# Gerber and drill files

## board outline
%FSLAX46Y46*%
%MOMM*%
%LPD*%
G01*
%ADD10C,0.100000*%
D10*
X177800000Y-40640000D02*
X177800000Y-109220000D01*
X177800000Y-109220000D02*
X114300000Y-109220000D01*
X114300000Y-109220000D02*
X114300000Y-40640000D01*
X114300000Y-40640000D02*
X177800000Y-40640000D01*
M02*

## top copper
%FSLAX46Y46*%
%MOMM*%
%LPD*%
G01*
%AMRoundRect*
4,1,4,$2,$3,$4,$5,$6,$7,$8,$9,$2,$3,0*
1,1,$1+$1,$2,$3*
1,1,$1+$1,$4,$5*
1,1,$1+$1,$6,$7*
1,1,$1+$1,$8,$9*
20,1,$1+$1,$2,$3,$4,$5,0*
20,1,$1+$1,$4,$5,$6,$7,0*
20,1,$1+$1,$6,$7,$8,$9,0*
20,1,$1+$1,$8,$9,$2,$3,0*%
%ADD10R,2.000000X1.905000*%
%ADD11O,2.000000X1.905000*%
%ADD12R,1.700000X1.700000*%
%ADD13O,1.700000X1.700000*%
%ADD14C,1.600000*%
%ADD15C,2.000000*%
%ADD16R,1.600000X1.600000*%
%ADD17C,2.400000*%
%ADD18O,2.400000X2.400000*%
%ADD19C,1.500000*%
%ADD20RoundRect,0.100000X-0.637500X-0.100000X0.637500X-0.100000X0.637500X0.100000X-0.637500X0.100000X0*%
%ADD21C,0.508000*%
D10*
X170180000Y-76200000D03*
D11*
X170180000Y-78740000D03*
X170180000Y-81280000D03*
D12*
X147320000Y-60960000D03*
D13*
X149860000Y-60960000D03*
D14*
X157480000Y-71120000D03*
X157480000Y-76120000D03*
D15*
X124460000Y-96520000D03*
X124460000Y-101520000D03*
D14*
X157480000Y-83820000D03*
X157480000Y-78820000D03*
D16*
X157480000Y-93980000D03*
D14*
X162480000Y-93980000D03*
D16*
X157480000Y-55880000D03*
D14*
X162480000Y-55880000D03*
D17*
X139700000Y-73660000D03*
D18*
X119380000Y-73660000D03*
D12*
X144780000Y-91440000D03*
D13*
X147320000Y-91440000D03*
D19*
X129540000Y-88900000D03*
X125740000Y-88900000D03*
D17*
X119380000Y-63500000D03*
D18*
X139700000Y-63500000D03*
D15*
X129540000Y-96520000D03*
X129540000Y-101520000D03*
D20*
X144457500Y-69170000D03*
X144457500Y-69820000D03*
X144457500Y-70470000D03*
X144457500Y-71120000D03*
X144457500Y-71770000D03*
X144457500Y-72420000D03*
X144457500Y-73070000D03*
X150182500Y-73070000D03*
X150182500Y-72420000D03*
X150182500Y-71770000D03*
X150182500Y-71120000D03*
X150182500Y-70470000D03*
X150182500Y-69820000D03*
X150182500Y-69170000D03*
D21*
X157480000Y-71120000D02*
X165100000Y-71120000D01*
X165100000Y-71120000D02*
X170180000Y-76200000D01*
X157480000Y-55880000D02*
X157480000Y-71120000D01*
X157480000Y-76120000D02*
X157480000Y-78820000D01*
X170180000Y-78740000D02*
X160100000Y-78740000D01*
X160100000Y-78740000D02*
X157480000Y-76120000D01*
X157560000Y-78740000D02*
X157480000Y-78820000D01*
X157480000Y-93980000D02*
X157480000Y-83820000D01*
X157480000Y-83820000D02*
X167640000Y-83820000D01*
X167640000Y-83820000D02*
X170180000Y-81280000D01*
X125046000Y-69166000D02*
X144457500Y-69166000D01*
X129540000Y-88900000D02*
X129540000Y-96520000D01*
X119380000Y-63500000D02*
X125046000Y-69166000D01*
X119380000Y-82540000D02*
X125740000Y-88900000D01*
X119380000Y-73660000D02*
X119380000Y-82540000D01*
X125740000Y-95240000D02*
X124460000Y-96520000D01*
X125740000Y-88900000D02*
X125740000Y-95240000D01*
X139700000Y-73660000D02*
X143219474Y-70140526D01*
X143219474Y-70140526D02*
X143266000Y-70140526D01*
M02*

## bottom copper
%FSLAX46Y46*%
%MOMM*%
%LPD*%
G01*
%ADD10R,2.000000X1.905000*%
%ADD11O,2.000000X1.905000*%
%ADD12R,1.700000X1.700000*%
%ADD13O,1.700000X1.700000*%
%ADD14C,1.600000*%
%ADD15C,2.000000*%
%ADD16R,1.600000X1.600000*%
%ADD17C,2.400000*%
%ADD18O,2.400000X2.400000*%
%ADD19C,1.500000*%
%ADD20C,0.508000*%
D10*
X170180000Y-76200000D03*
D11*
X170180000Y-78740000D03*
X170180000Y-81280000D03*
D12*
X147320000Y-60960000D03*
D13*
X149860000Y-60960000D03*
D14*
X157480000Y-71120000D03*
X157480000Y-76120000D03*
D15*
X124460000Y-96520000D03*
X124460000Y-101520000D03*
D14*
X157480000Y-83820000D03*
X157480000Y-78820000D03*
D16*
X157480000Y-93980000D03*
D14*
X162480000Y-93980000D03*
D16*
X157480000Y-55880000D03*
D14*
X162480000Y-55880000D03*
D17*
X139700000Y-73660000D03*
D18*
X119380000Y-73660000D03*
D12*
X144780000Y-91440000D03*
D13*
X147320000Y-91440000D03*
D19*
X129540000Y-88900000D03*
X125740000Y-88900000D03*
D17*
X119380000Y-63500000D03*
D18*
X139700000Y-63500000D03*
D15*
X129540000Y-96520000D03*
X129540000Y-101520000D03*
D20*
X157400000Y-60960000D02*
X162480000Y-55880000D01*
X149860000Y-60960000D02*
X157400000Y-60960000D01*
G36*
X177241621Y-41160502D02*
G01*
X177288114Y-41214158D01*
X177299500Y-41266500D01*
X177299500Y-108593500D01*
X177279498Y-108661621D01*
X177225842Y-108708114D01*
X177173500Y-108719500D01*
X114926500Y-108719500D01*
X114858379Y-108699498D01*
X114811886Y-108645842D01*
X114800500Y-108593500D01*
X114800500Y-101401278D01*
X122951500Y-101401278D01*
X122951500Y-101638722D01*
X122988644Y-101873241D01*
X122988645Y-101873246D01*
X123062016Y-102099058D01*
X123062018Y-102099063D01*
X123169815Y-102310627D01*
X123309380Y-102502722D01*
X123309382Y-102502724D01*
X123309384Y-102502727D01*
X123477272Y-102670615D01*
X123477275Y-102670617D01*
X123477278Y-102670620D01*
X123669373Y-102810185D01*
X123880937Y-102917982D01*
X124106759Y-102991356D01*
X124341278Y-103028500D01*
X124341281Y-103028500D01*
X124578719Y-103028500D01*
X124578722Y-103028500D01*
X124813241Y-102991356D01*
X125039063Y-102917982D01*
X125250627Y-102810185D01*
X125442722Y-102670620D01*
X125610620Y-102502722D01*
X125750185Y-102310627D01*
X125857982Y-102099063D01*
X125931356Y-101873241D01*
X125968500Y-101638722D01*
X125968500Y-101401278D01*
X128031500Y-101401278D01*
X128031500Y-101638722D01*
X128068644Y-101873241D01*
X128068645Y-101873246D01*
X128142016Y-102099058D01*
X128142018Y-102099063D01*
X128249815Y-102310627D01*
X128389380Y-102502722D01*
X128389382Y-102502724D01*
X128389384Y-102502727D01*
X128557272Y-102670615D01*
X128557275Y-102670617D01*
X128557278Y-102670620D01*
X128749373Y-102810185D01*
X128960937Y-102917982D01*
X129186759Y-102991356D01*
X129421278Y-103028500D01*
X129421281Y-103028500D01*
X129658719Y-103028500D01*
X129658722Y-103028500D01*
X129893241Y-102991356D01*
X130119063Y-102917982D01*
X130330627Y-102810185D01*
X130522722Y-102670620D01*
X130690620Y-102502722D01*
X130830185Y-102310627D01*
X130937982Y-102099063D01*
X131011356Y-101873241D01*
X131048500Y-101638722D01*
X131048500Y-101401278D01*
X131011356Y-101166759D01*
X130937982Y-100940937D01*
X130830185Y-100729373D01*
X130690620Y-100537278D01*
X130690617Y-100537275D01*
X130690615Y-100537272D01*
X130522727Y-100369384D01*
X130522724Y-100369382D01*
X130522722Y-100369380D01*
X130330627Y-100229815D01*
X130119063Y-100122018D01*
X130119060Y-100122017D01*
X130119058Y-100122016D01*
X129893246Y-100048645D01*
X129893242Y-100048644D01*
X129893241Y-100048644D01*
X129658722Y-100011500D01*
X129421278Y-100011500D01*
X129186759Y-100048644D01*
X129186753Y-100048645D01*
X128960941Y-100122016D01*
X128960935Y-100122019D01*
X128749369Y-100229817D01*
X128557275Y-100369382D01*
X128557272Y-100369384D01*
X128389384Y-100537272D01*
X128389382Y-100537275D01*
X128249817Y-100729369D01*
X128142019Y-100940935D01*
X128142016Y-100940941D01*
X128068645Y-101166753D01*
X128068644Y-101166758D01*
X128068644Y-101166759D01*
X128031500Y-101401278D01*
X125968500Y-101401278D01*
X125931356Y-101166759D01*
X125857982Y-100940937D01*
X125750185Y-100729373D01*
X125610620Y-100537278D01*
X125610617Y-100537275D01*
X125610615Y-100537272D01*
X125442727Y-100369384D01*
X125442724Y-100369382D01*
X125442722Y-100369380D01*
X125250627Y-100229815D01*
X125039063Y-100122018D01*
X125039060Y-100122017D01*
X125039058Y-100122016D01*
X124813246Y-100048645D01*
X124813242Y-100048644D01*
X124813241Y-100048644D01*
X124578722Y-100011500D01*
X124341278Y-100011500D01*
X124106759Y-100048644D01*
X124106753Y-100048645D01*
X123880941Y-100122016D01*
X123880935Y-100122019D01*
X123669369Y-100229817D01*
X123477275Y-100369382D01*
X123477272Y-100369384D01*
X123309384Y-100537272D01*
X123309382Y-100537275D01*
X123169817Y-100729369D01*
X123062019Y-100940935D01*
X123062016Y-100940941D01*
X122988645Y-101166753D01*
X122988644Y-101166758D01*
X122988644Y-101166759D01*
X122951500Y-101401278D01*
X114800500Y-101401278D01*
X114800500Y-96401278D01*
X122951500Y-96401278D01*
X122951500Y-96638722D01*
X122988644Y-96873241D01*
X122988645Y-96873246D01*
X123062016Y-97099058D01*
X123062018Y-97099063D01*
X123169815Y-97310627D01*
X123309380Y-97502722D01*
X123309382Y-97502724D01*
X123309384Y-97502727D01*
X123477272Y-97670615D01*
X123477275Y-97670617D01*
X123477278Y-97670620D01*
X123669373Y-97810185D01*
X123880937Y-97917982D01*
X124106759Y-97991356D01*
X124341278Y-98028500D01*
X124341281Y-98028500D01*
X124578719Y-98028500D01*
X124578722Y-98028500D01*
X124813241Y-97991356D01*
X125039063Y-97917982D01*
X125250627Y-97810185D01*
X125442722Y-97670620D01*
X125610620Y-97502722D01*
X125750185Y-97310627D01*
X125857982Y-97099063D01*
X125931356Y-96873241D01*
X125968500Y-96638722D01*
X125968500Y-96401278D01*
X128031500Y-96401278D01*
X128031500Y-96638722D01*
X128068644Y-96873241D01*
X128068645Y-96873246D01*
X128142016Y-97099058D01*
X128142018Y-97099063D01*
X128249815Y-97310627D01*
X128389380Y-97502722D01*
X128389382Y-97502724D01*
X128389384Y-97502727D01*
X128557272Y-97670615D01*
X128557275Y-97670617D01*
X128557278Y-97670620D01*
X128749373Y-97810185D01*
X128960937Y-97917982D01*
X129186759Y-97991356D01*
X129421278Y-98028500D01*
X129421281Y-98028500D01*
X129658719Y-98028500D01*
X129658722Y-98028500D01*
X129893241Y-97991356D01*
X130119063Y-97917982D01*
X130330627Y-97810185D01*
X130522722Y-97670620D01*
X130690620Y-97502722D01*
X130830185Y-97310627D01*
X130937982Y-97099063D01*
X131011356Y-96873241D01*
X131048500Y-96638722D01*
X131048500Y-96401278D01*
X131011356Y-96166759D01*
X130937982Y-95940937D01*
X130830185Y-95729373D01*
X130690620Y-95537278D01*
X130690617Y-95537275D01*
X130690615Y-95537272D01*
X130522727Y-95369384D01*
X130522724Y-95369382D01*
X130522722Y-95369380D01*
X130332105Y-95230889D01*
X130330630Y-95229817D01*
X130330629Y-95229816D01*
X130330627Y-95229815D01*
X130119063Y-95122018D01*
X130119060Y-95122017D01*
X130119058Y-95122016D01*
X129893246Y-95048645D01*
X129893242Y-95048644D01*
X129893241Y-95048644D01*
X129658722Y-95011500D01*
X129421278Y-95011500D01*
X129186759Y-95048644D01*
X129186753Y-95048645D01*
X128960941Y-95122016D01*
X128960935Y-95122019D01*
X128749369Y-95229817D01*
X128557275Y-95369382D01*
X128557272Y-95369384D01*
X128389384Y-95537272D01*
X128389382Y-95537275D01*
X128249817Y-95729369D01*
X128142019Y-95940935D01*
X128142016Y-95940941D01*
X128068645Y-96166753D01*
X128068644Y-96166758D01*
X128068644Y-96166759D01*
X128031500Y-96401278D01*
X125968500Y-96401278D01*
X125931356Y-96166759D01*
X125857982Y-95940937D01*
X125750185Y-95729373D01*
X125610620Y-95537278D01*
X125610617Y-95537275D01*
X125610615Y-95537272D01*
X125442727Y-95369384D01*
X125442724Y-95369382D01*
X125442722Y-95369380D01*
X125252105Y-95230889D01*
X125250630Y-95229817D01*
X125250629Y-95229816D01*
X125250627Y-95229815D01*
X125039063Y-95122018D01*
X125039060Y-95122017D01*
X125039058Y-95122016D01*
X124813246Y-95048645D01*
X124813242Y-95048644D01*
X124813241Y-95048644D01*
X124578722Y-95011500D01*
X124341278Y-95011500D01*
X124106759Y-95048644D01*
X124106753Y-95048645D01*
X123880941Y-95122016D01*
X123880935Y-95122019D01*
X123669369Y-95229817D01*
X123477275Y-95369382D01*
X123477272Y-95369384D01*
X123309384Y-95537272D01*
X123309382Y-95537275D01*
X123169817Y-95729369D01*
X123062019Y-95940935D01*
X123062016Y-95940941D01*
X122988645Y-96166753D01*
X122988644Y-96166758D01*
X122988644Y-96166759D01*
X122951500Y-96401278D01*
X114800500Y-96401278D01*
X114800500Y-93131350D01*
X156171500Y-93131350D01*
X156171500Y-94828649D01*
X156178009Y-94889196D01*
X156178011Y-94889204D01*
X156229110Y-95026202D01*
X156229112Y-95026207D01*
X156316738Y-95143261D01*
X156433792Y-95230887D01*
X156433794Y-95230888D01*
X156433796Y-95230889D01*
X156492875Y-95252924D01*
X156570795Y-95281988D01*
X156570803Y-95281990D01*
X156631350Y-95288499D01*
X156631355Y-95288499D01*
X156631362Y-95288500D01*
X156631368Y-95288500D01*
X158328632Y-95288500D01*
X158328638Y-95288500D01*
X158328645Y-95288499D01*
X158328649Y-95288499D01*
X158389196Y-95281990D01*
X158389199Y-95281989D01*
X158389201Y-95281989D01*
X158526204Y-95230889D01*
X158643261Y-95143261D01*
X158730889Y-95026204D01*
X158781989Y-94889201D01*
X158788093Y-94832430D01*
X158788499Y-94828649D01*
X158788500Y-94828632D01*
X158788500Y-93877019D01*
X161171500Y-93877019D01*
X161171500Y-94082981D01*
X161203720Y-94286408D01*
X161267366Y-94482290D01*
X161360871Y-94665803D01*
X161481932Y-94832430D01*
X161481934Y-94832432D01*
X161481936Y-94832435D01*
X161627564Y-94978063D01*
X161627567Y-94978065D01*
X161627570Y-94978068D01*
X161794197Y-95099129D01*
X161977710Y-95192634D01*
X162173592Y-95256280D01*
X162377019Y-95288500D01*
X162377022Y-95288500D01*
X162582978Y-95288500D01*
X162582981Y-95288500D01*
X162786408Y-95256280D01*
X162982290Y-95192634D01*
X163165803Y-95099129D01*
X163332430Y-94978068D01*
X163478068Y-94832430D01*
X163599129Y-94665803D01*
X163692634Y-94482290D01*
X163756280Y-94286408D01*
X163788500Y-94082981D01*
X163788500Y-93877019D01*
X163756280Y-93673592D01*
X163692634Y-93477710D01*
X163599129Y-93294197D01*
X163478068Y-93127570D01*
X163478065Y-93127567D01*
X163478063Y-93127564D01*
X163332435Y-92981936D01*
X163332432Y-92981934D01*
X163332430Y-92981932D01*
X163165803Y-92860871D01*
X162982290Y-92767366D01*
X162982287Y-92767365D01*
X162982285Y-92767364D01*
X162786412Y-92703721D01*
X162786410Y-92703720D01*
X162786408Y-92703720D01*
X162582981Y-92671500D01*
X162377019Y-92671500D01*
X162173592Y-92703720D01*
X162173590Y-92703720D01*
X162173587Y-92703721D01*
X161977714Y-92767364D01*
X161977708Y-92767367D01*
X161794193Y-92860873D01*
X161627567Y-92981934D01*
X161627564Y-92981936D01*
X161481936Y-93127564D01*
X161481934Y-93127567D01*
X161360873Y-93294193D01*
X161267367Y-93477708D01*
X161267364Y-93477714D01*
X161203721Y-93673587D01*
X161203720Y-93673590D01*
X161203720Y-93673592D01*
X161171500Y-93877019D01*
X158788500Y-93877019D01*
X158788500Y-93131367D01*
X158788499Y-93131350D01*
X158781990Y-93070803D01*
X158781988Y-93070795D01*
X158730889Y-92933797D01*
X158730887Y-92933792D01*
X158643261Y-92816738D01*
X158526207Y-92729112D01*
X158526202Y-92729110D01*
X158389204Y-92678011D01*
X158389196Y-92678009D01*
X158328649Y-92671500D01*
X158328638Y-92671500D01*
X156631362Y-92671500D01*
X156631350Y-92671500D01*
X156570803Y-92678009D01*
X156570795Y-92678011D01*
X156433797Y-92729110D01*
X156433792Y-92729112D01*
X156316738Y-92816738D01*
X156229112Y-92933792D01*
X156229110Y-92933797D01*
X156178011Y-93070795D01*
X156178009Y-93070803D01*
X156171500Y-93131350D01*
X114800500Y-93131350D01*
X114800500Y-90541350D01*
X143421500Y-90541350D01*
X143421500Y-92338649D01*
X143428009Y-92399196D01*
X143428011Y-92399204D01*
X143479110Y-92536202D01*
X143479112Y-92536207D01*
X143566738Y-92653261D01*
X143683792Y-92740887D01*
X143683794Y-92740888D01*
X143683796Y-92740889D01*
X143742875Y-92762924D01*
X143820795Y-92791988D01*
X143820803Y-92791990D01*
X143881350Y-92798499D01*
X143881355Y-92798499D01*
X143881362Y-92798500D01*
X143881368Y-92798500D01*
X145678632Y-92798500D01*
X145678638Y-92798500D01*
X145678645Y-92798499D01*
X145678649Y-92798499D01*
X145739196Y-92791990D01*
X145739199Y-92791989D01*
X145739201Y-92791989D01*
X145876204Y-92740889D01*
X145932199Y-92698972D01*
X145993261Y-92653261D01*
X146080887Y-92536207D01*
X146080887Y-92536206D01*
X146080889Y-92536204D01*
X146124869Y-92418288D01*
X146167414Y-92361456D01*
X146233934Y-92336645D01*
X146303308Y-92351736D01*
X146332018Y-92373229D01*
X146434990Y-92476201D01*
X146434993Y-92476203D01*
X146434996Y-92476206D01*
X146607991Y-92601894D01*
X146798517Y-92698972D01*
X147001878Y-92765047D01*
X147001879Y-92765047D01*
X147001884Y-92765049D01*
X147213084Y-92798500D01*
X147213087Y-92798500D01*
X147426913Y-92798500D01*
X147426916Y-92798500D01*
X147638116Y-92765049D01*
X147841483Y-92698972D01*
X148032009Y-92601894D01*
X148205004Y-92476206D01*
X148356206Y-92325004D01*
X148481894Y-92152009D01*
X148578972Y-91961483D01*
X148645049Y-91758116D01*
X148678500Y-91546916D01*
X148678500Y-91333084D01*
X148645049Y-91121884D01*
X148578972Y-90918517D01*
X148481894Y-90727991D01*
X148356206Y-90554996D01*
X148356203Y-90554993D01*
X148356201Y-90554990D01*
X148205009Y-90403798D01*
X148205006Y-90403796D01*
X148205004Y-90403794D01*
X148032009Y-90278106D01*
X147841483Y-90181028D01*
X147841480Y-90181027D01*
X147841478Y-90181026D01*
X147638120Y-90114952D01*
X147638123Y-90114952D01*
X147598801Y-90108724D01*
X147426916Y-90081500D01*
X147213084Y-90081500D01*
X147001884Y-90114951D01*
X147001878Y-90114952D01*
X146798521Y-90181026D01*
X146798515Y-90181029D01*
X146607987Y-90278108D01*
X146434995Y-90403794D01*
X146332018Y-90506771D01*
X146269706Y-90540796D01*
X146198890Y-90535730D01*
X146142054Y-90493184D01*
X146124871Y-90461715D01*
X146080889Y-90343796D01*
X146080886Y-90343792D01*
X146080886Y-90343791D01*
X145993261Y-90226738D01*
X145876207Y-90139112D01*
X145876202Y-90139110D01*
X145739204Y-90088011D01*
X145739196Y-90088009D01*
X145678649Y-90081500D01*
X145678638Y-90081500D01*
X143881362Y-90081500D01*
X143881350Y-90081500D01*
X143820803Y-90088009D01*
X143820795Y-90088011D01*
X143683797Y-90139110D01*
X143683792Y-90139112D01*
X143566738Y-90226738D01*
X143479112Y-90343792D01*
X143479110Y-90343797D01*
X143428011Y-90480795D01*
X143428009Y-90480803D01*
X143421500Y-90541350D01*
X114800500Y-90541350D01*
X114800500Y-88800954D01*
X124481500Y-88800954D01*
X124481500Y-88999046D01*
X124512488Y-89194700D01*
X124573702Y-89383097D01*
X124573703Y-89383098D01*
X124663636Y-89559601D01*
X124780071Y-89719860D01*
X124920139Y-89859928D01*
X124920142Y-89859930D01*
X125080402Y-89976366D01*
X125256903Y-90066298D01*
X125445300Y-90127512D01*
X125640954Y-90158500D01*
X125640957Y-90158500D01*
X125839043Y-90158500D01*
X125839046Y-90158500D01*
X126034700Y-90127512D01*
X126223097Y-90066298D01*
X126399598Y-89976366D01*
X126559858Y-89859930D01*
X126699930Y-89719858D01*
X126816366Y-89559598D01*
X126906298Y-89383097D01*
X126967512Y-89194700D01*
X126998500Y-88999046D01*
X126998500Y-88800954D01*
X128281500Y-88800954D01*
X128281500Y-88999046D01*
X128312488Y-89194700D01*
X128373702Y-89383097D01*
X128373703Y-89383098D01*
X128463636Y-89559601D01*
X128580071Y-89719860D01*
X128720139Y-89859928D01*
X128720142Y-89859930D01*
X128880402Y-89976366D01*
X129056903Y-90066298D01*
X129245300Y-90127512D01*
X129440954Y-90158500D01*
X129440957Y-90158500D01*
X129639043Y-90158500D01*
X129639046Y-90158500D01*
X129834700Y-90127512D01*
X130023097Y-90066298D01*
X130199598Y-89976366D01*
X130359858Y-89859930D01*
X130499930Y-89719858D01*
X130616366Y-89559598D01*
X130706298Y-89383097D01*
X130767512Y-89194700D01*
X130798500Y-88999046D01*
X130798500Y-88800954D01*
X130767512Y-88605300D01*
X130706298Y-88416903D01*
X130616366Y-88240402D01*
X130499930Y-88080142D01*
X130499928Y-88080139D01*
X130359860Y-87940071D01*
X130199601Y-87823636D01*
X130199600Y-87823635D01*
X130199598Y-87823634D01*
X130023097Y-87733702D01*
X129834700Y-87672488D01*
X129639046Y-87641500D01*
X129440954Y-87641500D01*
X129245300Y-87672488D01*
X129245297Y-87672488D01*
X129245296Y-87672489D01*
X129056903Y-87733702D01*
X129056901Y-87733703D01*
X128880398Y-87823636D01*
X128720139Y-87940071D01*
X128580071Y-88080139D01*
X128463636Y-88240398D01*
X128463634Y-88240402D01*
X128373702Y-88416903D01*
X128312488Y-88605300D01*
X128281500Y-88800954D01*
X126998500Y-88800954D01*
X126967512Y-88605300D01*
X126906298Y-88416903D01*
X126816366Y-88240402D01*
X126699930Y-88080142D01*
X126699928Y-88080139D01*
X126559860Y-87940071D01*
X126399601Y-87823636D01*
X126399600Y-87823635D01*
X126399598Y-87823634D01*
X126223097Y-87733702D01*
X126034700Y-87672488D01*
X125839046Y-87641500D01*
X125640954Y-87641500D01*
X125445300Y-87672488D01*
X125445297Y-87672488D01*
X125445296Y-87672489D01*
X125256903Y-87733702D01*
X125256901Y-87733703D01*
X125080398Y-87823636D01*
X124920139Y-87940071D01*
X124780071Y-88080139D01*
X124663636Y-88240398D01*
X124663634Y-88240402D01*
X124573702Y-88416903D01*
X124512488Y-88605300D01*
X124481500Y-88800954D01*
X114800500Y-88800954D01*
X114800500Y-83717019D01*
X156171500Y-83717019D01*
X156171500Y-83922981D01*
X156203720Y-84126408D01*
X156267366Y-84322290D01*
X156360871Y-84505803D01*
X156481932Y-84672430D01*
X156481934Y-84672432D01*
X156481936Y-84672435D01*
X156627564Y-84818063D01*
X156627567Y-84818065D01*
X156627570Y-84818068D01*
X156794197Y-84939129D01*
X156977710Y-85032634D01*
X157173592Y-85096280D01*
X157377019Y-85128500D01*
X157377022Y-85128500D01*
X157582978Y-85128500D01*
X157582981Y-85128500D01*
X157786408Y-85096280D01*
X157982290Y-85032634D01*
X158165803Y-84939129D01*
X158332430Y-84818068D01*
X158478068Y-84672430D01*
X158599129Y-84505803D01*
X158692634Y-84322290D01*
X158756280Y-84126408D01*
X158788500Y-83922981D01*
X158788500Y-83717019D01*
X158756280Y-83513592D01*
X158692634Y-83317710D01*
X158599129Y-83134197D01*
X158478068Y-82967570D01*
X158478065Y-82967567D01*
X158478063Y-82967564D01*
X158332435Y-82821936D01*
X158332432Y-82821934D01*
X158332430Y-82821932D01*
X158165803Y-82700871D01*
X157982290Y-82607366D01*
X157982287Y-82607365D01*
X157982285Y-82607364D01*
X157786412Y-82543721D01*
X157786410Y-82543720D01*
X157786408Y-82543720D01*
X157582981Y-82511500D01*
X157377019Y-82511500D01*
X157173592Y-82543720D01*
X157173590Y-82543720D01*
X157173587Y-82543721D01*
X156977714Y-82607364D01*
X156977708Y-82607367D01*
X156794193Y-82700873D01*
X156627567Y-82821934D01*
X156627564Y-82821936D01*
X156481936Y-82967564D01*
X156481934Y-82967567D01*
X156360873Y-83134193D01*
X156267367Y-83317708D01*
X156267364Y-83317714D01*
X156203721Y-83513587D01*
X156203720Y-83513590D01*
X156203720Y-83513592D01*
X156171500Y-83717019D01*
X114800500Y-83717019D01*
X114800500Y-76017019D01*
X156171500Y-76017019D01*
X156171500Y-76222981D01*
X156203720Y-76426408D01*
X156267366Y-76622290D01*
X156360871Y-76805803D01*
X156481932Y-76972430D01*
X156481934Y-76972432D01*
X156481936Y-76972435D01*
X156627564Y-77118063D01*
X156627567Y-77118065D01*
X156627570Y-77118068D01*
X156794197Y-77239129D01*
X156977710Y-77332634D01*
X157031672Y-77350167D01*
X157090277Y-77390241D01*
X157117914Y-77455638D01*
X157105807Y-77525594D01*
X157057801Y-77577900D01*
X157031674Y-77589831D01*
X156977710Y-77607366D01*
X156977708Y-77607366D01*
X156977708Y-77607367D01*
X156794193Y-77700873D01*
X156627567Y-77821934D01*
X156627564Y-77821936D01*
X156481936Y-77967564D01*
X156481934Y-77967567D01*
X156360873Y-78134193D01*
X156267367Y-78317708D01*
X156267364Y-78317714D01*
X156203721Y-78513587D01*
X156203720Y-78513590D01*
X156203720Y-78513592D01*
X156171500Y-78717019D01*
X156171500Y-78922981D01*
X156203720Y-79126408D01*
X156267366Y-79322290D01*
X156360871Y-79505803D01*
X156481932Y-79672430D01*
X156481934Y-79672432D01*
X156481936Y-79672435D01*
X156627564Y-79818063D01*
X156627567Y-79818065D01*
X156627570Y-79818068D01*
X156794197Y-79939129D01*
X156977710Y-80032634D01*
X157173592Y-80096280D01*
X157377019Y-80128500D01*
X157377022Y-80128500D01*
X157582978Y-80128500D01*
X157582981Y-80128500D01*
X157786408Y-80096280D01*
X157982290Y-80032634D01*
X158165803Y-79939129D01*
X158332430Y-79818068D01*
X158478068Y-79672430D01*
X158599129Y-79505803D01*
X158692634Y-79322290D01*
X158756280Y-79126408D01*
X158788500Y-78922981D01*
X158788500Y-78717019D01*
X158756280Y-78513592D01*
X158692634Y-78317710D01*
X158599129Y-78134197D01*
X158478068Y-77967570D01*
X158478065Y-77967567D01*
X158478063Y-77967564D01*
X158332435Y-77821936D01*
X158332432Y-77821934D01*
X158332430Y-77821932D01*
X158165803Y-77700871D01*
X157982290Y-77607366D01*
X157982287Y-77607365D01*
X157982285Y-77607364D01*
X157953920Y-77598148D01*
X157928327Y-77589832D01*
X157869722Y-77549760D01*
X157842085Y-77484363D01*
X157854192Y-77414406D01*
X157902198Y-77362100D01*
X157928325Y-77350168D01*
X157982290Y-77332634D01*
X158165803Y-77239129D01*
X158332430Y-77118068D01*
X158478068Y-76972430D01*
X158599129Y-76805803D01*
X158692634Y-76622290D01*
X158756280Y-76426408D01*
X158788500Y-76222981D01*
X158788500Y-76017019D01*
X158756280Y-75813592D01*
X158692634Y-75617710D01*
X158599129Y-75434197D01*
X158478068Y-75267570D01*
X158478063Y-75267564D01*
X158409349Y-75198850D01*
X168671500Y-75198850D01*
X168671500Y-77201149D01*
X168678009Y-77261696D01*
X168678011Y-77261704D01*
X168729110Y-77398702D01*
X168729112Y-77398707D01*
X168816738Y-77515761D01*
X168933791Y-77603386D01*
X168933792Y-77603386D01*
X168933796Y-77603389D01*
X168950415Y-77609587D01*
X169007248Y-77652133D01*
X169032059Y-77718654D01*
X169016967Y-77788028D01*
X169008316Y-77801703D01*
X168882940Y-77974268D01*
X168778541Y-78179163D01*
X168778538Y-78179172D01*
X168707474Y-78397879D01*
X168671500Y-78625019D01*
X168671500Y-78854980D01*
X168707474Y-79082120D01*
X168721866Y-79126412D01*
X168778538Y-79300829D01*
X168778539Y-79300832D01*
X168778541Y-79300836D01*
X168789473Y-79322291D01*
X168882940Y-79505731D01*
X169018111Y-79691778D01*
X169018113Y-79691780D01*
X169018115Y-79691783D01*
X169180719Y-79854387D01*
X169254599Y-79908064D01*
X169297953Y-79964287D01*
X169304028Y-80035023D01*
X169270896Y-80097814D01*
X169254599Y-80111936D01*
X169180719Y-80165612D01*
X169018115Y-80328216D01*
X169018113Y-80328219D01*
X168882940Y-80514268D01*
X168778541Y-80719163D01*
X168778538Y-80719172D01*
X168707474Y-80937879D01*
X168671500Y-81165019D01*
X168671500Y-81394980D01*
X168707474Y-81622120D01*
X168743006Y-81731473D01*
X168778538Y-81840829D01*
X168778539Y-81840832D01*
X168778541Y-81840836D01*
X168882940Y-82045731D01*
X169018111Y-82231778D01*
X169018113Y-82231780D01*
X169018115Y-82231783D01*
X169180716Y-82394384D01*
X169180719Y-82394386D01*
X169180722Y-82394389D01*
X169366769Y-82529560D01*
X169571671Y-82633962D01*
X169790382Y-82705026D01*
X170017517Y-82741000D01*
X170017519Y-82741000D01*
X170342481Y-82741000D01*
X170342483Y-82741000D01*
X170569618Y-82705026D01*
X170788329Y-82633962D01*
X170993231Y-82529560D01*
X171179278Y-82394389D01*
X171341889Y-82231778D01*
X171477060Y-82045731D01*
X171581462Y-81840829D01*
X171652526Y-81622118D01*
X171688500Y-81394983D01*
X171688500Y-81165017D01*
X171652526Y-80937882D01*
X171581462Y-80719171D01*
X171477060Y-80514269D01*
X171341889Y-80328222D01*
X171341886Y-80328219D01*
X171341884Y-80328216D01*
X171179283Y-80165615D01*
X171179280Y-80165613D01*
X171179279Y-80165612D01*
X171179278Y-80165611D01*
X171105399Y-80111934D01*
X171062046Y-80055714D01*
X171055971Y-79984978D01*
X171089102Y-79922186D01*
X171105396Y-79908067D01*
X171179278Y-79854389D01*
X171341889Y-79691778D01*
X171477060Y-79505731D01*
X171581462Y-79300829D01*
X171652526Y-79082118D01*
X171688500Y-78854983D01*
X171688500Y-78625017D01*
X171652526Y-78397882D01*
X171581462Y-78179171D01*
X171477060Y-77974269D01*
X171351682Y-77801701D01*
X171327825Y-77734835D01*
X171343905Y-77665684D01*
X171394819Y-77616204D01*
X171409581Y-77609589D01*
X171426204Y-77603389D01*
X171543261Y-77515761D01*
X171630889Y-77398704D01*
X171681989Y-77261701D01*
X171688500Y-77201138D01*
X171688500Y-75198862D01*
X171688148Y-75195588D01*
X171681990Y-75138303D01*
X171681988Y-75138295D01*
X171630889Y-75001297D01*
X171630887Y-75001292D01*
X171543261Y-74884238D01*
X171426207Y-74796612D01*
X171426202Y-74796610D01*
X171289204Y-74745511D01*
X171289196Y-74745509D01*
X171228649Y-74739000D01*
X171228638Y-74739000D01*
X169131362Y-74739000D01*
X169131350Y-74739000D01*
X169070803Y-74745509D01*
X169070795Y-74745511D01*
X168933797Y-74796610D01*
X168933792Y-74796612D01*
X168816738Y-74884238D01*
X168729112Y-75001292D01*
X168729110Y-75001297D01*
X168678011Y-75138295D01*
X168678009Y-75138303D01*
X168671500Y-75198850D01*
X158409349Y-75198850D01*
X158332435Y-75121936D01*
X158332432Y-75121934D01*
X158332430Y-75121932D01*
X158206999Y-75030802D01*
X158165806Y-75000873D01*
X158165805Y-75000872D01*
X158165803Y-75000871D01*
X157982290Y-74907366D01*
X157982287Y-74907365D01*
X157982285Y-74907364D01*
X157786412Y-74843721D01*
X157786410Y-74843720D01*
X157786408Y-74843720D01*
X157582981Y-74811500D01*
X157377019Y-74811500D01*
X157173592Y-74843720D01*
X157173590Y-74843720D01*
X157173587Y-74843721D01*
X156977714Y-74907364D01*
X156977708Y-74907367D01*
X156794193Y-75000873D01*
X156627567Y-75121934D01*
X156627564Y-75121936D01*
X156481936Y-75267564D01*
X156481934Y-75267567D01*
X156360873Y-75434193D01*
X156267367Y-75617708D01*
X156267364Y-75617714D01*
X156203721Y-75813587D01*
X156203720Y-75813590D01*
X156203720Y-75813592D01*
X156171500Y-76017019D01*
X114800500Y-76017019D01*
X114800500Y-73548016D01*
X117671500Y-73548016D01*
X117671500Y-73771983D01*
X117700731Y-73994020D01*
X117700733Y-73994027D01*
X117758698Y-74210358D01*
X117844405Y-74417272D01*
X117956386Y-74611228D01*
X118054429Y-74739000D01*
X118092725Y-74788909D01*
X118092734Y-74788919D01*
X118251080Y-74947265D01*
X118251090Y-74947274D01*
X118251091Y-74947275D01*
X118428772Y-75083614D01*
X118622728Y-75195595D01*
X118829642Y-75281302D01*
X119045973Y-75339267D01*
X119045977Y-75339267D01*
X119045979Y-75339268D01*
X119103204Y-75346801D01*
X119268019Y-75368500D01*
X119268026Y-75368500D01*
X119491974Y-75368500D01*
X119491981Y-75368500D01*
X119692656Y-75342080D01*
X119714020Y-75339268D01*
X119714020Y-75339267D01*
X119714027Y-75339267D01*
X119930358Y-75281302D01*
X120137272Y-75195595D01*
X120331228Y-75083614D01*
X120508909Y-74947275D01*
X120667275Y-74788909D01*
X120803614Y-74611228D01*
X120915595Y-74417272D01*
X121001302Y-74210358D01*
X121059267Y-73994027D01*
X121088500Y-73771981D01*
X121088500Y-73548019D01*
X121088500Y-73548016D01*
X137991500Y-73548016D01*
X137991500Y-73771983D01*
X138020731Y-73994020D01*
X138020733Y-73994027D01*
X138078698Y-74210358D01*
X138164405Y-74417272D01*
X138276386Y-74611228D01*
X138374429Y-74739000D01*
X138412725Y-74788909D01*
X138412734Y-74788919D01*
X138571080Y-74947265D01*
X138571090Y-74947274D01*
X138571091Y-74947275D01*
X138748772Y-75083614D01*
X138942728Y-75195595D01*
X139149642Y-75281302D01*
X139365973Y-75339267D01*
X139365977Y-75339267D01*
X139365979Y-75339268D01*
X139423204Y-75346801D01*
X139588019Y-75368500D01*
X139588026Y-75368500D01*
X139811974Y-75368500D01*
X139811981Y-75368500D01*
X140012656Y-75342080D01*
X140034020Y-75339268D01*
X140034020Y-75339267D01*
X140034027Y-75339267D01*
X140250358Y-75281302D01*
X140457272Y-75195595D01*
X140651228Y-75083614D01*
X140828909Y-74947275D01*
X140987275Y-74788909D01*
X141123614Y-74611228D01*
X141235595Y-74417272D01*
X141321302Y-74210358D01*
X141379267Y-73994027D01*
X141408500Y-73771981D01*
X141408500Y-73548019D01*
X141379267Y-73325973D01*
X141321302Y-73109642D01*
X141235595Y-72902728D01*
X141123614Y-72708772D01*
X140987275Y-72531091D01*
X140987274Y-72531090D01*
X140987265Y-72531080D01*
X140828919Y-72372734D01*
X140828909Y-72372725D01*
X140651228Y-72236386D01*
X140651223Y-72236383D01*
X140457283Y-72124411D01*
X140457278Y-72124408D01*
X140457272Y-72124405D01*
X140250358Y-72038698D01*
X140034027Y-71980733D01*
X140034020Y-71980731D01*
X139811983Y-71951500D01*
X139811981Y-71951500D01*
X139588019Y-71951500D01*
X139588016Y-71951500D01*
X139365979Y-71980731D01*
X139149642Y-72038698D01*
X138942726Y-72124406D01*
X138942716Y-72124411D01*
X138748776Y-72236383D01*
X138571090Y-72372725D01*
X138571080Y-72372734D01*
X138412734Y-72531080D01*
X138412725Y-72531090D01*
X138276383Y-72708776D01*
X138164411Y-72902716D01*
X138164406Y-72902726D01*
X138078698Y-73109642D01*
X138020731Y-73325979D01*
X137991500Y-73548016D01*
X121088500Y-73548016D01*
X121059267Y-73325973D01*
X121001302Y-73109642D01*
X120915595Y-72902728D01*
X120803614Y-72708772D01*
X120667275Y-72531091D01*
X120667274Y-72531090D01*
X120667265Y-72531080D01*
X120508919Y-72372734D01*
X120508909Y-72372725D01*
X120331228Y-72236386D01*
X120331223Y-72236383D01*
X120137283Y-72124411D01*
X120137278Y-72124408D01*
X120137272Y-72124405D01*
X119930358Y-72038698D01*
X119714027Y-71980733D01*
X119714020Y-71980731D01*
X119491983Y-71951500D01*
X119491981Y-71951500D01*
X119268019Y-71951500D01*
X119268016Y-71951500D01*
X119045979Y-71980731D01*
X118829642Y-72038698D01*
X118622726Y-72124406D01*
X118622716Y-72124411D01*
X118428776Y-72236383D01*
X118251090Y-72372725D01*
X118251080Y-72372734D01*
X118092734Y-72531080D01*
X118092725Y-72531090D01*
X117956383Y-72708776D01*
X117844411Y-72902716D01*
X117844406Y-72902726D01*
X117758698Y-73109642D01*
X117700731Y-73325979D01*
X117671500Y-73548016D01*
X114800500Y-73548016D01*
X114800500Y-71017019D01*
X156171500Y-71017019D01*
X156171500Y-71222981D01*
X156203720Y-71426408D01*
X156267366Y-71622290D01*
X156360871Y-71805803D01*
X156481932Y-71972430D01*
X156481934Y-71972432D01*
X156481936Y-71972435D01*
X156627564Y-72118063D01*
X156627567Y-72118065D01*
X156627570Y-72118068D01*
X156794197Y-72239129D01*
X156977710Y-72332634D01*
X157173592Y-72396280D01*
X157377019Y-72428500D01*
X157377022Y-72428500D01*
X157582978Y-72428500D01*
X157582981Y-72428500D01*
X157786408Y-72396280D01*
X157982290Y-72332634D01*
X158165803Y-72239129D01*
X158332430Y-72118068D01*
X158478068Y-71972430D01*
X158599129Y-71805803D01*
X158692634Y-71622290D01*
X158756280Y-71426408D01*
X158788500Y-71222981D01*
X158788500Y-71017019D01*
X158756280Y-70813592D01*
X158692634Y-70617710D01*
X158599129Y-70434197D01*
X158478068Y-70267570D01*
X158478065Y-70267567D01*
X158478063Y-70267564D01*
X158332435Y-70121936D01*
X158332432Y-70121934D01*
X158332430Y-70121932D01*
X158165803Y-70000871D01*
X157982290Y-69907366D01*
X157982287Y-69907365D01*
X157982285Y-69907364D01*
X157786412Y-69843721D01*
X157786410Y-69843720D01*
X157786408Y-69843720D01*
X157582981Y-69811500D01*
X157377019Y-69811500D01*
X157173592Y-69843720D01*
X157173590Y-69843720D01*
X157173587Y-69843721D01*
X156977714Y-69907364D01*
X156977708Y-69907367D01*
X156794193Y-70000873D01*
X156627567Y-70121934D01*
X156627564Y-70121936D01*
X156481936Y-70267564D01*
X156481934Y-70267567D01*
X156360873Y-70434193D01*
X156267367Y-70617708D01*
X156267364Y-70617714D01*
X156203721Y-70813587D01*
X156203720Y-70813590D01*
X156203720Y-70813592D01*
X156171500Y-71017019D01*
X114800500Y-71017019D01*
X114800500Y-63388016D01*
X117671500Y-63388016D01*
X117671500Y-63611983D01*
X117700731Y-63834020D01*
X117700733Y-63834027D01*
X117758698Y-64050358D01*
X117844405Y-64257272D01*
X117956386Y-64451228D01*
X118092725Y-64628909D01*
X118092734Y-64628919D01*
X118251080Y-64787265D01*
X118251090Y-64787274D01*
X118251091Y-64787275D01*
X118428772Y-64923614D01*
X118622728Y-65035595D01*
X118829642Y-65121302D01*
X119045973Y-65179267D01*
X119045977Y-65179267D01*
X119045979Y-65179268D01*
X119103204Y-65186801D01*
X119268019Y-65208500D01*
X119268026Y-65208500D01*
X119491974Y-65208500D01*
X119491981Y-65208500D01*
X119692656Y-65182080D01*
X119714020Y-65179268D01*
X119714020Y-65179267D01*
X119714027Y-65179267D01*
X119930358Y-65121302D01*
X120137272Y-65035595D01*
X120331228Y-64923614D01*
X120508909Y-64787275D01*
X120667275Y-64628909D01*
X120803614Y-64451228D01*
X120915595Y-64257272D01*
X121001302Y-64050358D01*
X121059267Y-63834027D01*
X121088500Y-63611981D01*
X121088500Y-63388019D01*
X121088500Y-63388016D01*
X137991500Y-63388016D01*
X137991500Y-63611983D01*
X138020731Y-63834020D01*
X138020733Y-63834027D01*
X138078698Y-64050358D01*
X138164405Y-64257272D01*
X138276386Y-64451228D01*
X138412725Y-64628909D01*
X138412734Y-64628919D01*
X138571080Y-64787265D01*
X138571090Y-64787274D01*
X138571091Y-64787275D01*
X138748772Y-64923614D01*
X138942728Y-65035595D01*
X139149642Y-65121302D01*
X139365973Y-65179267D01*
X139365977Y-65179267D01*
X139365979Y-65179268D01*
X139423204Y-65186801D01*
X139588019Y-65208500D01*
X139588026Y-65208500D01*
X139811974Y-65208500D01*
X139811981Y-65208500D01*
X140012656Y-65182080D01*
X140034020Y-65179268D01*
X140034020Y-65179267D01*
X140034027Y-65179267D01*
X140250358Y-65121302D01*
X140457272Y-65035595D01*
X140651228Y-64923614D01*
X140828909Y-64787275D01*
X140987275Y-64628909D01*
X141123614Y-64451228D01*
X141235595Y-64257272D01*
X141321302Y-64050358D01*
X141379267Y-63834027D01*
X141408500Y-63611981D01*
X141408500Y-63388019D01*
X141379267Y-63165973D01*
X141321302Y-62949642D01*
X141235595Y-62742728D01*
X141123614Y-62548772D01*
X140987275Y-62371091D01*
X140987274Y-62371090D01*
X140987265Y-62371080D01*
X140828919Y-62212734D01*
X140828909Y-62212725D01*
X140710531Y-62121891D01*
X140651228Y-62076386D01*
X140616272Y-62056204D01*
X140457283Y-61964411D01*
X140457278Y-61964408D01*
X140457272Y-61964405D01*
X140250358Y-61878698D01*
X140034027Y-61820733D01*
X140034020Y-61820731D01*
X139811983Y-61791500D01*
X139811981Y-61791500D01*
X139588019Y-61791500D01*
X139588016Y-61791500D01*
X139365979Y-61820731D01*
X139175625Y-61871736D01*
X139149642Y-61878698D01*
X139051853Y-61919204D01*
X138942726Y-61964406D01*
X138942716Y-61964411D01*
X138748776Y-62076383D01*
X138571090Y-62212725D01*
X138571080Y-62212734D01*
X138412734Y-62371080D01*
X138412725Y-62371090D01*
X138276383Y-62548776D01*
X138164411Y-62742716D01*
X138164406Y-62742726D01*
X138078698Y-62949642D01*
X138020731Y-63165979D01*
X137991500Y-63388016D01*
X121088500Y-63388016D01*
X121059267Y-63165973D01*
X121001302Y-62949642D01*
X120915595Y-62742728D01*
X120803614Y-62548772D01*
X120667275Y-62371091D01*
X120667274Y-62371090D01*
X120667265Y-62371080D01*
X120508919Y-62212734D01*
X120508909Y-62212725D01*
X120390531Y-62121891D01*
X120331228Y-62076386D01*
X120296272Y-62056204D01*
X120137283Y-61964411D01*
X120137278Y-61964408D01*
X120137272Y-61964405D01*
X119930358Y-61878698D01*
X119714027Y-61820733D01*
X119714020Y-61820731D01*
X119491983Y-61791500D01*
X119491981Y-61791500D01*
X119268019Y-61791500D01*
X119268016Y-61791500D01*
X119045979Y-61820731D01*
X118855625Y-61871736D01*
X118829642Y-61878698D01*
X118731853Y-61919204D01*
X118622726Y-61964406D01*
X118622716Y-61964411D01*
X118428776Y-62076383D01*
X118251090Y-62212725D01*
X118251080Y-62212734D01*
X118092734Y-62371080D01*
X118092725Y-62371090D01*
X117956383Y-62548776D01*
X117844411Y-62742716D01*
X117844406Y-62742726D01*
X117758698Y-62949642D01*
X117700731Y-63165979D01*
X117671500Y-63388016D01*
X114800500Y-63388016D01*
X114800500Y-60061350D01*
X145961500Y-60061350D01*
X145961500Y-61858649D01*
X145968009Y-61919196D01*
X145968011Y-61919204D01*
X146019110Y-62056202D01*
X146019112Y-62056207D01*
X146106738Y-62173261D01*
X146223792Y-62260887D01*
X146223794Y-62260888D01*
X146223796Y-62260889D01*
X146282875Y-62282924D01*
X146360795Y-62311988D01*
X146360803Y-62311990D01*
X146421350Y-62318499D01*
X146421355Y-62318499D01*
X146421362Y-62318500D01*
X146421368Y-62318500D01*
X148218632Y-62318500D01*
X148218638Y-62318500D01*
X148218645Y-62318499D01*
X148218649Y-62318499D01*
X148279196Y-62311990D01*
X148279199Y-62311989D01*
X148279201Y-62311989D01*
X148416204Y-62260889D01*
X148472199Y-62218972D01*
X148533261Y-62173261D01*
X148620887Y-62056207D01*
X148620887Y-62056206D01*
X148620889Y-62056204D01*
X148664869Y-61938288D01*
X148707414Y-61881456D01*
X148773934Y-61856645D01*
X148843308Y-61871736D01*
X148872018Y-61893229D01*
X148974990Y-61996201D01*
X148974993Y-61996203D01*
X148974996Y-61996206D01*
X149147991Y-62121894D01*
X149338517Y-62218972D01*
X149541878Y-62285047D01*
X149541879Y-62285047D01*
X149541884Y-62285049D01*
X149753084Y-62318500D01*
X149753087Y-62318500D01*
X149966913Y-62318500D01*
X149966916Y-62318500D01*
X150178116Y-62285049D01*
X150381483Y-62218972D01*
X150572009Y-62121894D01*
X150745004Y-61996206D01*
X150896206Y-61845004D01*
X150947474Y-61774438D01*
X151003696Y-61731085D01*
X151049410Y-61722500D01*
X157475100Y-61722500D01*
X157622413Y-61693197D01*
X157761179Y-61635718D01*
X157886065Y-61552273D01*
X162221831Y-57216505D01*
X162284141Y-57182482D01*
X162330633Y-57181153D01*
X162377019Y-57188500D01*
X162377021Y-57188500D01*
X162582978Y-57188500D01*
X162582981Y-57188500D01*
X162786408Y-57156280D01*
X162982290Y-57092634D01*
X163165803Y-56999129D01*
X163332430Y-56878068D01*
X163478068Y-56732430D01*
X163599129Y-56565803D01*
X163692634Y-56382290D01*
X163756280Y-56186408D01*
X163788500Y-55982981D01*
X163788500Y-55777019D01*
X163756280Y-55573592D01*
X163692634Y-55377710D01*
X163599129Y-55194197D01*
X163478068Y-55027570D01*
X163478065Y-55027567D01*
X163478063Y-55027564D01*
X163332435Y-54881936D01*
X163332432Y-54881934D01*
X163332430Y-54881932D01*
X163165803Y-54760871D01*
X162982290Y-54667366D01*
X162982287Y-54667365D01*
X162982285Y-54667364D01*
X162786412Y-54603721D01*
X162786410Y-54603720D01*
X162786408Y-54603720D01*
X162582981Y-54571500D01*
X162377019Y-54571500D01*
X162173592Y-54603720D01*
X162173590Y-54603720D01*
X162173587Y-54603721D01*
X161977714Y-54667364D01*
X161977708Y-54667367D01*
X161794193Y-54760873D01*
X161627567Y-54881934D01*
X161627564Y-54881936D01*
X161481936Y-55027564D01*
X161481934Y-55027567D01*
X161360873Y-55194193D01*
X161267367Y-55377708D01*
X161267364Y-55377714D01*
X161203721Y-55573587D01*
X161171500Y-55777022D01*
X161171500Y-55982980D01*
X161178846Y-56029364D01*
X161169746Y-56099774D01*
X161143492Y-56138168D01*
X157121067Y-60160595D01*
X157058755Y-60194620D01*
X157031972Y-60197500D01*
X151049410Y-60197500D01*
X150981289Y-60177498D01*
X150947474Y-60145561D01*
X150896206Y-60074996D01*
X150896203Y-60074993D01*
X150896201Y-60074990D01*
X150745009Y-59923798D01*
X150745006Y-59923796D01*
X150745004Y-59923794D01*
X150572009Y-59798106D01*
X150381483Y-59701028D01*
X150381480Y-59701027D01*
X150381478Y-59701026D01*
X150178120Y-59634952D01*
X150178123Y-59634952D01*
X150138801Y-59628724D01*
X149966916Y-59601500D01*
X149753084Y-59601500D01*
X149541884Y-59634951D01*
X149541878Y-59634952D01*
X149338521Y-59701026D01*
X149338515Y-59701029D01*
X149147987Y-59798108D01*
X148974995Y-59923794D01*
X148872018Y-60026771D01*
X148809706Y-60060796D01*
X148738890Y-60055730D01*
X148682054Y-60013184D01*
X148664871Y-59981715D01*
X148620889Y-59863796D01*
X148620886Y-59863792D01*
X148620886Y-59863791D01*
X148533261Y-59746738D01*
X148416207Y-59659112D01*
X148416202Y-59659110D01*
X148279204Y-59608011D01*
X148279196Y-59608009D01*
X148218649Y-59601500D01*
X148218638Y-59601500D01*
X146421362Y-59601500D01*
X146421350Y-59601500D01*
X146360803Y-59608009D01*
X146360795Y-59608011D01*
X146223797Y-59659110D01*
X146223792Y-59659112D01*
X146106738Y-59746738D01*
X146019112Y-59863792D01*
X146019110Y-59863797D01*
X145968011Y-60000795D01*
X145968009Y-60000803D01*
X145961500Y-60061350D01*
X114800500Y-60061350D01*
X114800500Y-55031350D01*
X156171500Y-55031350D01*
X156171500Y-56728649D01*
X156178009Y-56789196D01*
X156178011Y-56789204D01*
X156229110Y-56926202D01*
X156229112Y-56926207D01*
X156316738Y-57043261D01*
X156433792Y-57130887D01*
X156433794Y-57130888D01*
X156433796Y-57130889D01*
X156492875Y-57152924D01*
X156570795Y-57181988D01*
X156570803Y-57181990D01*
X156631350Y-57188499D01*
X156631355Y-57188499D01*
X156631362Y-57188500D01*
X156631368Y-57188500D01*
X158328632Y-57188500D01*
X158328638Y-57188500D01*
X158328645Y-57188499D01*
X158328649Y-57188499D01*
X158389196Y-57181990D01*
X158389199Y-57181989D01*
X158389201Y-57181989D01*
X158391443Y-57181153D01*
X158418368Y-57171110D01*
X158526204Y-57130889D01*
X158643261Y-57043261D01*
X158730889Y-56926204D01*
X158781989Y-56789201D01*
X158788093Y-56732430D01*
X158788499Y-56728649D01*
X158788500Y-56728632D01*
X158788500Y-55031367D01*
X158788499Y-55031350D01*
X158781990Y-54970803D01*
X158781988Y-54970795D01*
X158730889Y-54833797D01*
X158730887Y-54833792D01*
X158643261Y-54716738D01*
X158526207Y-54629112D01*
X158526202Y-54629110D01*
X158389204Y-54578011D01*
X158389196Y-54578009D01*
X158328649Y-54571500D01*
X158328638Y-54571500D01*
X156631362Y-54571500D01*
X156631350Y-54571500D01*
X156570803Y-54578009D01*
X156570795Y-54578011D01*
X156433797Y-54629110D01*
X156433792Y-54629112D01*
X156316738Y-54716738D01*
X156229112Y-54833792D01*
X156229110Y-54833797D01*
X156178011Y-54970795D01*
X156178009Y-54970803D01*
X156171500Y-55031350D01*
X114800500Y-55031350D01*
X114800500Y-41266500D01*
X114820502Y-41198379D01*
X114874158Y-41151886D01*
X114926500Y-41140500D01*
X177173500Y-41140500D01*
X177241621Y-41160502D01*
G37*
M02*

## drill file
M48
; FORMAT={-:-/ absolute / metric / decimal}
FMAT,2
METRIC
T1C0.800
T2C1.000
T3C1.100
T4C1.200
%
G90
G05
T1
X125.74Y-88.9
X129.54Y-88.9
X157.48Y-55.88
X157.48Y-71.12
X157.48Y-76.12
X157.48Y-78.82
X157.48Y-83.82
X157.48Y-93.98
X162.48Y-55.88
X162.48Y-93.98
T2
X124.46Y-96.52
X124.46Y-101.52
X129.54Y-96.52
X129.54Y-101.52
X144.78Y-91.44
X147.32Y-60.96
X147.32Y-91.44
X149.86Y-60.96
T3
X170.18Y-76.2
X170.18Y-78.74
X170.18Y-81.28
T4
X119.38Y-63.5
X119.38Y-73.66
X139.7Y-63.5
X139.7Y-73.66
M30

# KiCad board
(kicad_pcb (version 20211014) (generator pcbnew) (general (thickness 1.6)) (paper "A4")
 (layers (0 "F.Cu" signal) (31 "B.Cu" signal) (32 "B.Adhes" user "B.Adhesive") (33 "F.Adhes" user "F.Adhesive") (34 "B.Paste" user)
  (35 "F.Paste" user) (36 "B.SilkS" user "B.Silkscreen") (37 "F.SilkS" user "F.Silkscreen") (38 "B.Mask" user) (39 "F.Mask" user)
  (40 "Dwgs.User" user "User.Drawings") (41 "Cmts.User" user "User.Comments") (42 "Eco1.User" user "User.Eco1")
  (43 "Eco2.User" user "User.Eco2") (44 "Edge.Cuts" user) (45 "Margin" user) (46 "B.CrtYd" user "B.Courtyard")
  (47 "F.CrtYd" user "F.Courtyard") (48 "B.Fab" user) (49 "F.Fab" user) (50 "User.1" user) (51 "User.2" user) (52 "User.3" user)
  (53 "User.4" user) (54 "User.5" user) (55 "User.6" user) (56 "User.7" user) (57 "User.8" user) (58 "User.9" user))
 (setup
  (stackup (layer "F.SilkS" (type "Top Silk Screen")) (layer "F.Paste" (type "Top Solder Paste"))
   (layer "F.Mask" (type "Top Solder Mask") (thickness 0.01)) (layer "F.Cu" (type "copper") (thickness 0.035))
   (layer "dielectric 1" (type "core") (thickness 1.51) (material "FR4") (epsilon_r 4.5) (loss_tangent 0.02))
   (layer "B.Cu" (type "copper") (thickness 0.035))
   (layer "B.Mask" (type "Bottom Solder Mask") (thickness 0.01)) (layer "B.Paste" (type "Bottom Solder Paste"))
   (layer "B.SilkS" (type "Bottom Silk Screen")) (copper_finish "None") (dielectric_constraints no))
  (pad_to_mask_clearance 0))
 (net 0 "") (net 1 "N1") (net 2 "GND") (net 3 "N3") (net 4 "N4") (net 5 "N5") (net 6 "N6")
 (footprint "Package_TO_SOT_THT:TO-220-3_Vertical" (layer "F.Cu") (at 170.18 76.2 -90)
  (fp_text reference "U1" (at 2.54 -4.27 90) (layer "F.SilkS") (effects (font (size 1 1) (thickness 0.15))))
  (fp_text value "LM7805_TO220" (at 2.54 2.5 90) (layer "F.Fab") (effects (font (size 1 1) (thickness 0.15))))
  (pad "1" thru_hole rect (at 0 0 270) (size 1.905 2) (drill 1.1) (layers *.Cu *.Mask) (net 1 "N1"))
  (pad "2" thru_hole oval (at 2.54 0 270) (size 1.905 2) (drill 1.1) (layers *.Cu *.Mask) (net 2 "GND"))
  (pad "3" thru_hole oval (at 5.08 0 270) (size 1.905 2) (drill 1.1) (layers *.Cu *.Mask) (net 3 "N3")))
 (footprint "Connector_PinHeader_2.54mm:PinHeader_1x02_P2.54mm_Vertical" (layer "F.Cu") (at 147.32 60.96 90)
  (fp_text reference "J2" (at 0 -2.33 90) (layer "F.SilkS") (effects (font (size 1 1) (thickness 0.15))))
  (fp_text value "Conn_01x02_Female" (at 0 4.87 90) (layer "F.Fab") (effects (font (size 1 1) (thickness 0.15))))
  (pad "1" thru_hole rect (at 0 0 90) (size 1.7 1.7) (drill 1) (layers *.Cu *.Mask) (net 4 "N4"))
  (pad "2" thru_hole oval (at 0 2.54 90) (size 1.7 1.7) (drill 1) (layers *.Cu *.Mask) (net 2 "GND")))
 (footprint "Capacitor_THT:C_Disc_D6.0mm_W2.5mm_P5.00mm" (layer "F.Cu") (at 157.48 71.12 -90)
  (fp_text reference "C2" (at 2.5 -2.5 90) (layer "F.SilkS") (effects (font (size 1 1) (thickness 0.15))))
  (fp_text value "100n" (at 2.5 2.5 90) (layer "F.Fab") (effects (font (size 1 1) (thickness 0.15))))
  (pad "1" thru_hole circle (at 0 0 270) (size 1.6 1.6) (drill 0.8) (layers *.Cu *.Mask) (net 1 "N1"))
  (pad "2" thru_hole circle (at 5 0 270) (size 1.6 1.6) (drill 0.8) (layers *.Cu *.Mask) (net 2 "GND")))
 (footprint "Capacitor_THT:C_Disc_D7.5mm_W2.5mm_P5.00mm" (layer "F.Cu") (at 124.46 96.52 -90)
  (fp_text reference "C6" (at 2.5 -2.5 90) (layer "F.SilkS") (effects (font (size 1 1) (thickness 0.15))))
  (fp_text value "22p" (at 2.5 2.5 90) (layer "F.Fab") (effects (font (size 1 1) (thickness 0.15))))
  (pad "1" thru_hole circle (at 0 0 270) (size 2 2) (drill 1) (layers *.Cu *.Mask) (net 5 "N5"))
  (pad "2" thru_hole circle (at 5 0 270) (size 2 2) (drill 1) (layers *.Cu *.Mask) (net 2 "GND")))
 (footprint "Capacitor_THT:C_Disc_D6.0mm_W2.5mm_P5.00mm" (layer "F.Cu") (at 157.48 83.82 90)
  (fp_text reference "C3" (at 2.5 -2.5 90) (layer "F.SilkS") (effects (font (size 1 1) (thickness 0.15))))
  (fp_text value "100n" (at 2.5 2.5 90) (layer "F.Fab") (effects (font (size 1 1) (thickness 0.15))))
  (pad "1" thru_hole circle (at 0 0 90) (size 1.6 1.6) (drill 0.8) (layers *.Cu *.Mask) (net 3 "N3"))
  (pad "2" thru_hole circle (at 5 0 90) (size 1.6 1.6) (drill 0.8) (layers *.Cu *.Mask) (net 2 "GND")))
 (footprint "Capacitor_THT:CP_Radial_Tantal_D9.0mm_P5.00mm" (layer "F.Cu") (at 157.48 93.98)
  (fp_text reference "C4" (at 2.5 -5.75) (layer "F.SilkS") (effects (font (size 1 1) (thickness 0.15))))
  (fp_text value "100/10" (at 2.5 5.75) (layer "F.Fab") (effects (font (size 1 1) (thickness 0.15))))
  (pad "1" thru_hole rect (at 0 0) (size 1.6 1.6) (drill 0.8) (layers *.Cu *.Mask) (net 3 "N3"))
  (pad "2" thru_hole circle (at 5 0) (size 1.6 1.6) (drill 0.8) (layers *.Cu *.Mask) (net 2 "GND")))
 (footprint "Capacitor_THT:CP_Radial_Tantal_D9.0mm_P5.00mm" (layer "F.Cu") (at 157.48 55.88)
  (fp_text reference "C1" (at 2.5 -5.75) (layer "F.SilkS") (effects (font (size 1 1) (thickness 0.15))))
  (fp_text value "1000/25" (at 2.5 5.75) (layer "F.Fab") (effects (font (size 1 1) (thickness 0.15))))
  (pad "1" thru_hole rect (at 0 0) (size 1.6 1.6) (drill 0.8) (layers *.Cu *.Mask) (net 1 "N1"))
  (pad "2" thru_hole circle (at 5 0) (size 1.6 1.6) (drill 0.8) (layers *.Cu *.Mask) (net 2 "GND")))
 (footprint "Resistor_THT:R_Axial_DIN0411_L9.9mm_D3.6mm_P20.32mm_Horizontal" (layer "F.Cu") (at 139.7 73.66 180)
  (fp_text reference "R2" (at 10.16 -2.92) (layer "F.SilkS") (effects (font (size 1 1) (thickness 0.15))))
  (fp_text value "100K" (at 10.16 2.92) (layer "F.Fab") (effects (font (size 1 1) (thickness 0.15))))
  (pad "1" thru_hole circle (at 0 0 180) (size 2.4 2.4) (drill 1.2) (layers *.Cu *.Mask) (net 4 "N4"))
  (pad "2" thru_hole oval (at 20.32 0 180) (size 2.4 2.4) (drill 1.2) (layers *.Cu *.Mask) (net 5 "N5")))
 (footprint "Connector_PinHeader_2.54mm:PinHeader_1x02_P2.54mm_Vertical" (layer "F.Cu") (at 144.78 91.44 90)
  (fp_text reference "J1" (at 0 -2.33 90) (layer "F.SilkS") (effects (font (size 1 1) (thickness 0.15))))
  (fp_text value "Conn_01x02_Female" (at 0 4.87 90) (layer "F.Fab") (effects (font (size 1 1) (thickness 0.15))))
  (pad "1" thru_hole rect (at 0 0 90) (size 1.7 1.7) (drill 1) (layers *.Cu *.Mask) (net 2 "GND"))
  (pad "2" thru_hole oval (at 0 2.54 90) (size 1.7 1.7) (drill 1) (layers *.Cu *.Mask) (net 1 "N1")))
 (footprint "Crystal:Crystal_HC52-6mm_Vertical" (layer "F.Cu") (at 129.54 88.9 180)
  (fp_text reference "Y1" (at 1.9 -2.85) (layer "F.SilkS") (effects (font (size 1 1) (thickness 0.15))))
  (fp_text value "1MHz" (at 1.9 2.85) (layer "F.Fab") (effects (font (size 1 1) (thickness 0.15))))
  (pad "1" thru_hole circle (at 0 0 180) (size 1.5 1.5) (drill 0.8) (layers *.Cu *.Mask) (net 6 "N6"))
  (pad "2" thru_hole circle (at 3.8 0 180) (size 1.5 1.5) (drill 0.8) (layers *.Cu *.Mask) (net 5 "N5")))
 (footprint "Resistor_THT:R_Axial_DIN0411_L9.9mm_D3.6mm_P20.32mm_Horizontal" (layer "F.Cu") (at 119.38 63.5)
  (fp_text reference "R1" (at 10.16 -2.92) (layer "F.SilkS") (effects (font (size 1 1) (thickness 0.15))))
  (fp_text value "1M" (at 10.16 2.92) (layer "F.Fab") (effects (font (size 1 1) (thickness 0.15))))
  (pad "1" thru_hole circle (at 0 0) (size 2.4 2.4) (drill 1.2) (layers *.Cu *.Mask) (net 6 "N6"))
  (pad "2" thru_hole oval (at 20.32 0) (size 2.4 2.4) (drill 1.2) (layers *.Cu *.Mask) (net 4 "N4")))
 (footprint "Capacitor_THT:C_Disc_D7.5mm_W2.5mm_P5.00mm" (layer "F.Cu") (at 129.54 96.52 -90)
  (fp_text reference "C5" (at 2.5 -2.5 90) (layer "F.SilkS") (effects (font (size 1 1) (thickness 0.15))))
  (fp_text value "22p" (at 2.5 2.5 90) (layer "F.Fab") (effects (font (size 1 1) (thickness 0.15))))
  (pad "1" thru_hole circle (at 0 0 270) (size 2 2) (drill 1) (layers *.Cu *.Mask) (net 6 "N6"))
  (pad "2" thru_hole circle (at 5 0 270) (size 2 2) (drill 1) (layers *.Cu *.Mask) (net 2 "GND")))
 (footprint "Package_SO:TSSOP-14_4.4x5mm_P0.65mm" (layer "F.Cu") (at 147.32 71.12)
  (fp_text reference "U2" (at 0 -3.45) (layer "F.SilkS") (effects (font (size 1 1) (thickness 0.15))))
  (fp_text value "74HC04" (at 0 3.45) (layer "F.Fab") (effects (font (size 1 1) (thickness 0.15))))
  (pad "1" smd roundrect (at -2.8625 -1.95) (size 1.475 0.4) (layers "F.Cu" "F.Paste" "F.Mask") (roundrect_rratio 0.25) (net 6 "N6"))
  (pad "2" smd roundrect (at -2.8625 -1.3) (size 1.475 0.4) (layers "F.Cu" "F.Paste" "F.Mask") (roundrect_rratio 0.25) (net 4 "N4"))
  (pad "3" smd roundrect (at -2.8625 -0.65) (size 1.475 0.4) (layers "F.Cu" "F.Paste" "F.Mask") (roundrect_rratio 0.25))
  (pad "4" smd roundrect (at -2.8625 0) (size 1.475 0.4) (layers "F.Cu" "F.Paste" "F.Mask") (roundrect_rratio 0.25))
  (pad "5" smd roundrect (at -2.8625 0.65) (size 1.475 0.4) (layers "F.Cu" "F.Paste" "F.Mask") (roundrect_rratio 0.25))
  (pad "6" smd roundrect (at -2.8625 1.3) (size 1.475 0.4) (layers "F.Cu" "F.Paste" "F.Mask") (roundrect_rratio 0.25))
  (pad "7" smd roundrect (at -2.8625 1.95) (size 1.475 0.4) (layers "F.Cu" "F.Paste" "F.Mask") (roundrect_rratio 0.25))
  (pad "8" smd roundrect (at 2.8625 1.95) (size 1.475 0.4) (layers "F.Cu" "F.Paste" "F.Mask") (roundrect_rratio 0.25))
  (pad "9" smd roundrect (at 2.8625 1.3) (size 1.475 0.4) (layers "F.Cu" "F.Paste" "F.Mask") (roundrect_rratio 0.25))
  (pad "10" smd roundrect (at 2.8625 0.65) (size 1.475 0.4) (layers "F.Cu" "F.Paste" "F.Mask") (roundrect_rratio 0.25))
  (pad "11" smd roundrect (at 2.8625 0) (size 1.475 0.4) (layers "F.Cu" "F.Paste" "F.Mask") (roundrect_rratio 0.25))
  (pad "12" smd roundrect (at 2.8625 -0.65) (size 1.475 0.4) (layers "F.Cu" "F.Paste" "F.Mask") (roundrect_rratio 0.25))
  (pad "13" smd roundrect (at 2.8625 -1.3) (size 1.475 0.4) (layers "F.Cu" "F.Paste" "F.Mask") (roundrect_rratio 0.25))
  (pad "14" smd roundrect (at 2.8625 -1.95) (size 1.475 0.4) (layers "F.Cu" "F.Paste" "F.Mask") (roundrect_rratio 0.25)))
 (gr_line (start 177.8 40.64) (end 177.8 109.22) (layer "Edge.Cuts") (width 0.1))
 (gr_line (start 177.8 109.22) (end 114.3 109.22) (layer "Edge.Cuts") (width 0.1))
 (gr_line (start 114.3 109.22) (end 114.3 40.64) (layer "Edge.Cuts") (width 0.1))
 (gr_line (start 114.3 40.64) (end 177.8 40.64) (layer "Edge.Cuts") (width 0.1))
 (segment (start 157.48 71.12) (end 165.1 71.12) (width 0.508) (layer "F.Cu") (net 1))
 (segment (start 165.1 71.12) (end 170.18 76.2) (width 0.508) (layer "F.Cu") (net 1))
 (segment (start 157.48 55.88) (end 157.48 71.12) (width 0.508) (layer "F.Cu") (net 1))
 (segment (start 157.48 76.12) (end 157.48 78.82) (width 0.508) (layer "F.Cu") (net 2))
 (segment (start 170.18 78.74) (end 160.1 78.74) (width 0.508) (layer "F.Cu") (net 2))
 (segment (start 160.1 78.74) (end 157.48 76.12) (width 0.508) (layer "F.Cu") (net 2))
 (segment (start 157.56 78.74) (end 157.48 78.82) (width 0.508) (layer "F.Cu") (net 2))
 (segment (start 157.4 60.96) (end 162.48 55.88) (width 0.508) (layer "B.Cu") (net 2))
 (segment (start 149.86 60.96) (end 157.4 60.96) (width 0.508) (layer "B.Cu") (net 2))
 (segment (start 157.48 93.98) (end 157.48 83.82) (width 0.508) (layer "F.Cu") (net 3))
 (segment (start 157.48 83.82) (end 167.64 83.82) (width 0.508) (layer "F.Cu") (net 3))
 (segment (start 167.64 83.82) (end 170.18 81.28) (width 0.508) (layer "F.Cu") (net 3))
 (segment (start 125.046 69.166) (end 144.4575 69.166) (width 0.508) (layer "F.Cu") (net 6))
 (segment (start 129.54 88.9) (end 129.54 96.52) (width 0.508) (layer "F.Cu") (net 6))
 (segment (start 119.38 63.5) (end 125.046 69.166) (width 0.508) (layer "F.Cu") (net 6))
 (segment (start 119.38 82.54) (end 125.74 88.9) (width 0.508) (layer "F.Cu") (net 5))
 (segment (start 119.38 73.66) (end 119.38 82.54) (width 0.508) (layer "F.Cu") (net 5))
 (segment (start 125.74 95.24) (end 124.46 96.52) (width 0.508) (layer "F.Cu") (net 5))
 (segment (start 125.74 88.9) (end 125.74 95.24) (width 0.508) (layer "F.Cu") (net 5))
 (segment (start 139.7 73.66) (end 143.219474 70.140526) (width 0.508) (layer "F.Cu") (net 4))
 (segment (start 143.219474 70.140526) (end 143.266 70.140526) (width 0.508) (layer "F.Cu") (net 4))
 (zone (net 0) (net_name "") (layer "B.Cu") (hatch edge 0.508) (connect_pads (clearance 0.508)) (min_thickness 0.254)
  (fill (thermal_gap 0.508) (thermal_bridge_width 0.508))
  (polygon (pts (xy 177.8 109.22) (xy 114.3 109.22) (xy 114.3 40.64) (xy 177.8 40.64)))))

